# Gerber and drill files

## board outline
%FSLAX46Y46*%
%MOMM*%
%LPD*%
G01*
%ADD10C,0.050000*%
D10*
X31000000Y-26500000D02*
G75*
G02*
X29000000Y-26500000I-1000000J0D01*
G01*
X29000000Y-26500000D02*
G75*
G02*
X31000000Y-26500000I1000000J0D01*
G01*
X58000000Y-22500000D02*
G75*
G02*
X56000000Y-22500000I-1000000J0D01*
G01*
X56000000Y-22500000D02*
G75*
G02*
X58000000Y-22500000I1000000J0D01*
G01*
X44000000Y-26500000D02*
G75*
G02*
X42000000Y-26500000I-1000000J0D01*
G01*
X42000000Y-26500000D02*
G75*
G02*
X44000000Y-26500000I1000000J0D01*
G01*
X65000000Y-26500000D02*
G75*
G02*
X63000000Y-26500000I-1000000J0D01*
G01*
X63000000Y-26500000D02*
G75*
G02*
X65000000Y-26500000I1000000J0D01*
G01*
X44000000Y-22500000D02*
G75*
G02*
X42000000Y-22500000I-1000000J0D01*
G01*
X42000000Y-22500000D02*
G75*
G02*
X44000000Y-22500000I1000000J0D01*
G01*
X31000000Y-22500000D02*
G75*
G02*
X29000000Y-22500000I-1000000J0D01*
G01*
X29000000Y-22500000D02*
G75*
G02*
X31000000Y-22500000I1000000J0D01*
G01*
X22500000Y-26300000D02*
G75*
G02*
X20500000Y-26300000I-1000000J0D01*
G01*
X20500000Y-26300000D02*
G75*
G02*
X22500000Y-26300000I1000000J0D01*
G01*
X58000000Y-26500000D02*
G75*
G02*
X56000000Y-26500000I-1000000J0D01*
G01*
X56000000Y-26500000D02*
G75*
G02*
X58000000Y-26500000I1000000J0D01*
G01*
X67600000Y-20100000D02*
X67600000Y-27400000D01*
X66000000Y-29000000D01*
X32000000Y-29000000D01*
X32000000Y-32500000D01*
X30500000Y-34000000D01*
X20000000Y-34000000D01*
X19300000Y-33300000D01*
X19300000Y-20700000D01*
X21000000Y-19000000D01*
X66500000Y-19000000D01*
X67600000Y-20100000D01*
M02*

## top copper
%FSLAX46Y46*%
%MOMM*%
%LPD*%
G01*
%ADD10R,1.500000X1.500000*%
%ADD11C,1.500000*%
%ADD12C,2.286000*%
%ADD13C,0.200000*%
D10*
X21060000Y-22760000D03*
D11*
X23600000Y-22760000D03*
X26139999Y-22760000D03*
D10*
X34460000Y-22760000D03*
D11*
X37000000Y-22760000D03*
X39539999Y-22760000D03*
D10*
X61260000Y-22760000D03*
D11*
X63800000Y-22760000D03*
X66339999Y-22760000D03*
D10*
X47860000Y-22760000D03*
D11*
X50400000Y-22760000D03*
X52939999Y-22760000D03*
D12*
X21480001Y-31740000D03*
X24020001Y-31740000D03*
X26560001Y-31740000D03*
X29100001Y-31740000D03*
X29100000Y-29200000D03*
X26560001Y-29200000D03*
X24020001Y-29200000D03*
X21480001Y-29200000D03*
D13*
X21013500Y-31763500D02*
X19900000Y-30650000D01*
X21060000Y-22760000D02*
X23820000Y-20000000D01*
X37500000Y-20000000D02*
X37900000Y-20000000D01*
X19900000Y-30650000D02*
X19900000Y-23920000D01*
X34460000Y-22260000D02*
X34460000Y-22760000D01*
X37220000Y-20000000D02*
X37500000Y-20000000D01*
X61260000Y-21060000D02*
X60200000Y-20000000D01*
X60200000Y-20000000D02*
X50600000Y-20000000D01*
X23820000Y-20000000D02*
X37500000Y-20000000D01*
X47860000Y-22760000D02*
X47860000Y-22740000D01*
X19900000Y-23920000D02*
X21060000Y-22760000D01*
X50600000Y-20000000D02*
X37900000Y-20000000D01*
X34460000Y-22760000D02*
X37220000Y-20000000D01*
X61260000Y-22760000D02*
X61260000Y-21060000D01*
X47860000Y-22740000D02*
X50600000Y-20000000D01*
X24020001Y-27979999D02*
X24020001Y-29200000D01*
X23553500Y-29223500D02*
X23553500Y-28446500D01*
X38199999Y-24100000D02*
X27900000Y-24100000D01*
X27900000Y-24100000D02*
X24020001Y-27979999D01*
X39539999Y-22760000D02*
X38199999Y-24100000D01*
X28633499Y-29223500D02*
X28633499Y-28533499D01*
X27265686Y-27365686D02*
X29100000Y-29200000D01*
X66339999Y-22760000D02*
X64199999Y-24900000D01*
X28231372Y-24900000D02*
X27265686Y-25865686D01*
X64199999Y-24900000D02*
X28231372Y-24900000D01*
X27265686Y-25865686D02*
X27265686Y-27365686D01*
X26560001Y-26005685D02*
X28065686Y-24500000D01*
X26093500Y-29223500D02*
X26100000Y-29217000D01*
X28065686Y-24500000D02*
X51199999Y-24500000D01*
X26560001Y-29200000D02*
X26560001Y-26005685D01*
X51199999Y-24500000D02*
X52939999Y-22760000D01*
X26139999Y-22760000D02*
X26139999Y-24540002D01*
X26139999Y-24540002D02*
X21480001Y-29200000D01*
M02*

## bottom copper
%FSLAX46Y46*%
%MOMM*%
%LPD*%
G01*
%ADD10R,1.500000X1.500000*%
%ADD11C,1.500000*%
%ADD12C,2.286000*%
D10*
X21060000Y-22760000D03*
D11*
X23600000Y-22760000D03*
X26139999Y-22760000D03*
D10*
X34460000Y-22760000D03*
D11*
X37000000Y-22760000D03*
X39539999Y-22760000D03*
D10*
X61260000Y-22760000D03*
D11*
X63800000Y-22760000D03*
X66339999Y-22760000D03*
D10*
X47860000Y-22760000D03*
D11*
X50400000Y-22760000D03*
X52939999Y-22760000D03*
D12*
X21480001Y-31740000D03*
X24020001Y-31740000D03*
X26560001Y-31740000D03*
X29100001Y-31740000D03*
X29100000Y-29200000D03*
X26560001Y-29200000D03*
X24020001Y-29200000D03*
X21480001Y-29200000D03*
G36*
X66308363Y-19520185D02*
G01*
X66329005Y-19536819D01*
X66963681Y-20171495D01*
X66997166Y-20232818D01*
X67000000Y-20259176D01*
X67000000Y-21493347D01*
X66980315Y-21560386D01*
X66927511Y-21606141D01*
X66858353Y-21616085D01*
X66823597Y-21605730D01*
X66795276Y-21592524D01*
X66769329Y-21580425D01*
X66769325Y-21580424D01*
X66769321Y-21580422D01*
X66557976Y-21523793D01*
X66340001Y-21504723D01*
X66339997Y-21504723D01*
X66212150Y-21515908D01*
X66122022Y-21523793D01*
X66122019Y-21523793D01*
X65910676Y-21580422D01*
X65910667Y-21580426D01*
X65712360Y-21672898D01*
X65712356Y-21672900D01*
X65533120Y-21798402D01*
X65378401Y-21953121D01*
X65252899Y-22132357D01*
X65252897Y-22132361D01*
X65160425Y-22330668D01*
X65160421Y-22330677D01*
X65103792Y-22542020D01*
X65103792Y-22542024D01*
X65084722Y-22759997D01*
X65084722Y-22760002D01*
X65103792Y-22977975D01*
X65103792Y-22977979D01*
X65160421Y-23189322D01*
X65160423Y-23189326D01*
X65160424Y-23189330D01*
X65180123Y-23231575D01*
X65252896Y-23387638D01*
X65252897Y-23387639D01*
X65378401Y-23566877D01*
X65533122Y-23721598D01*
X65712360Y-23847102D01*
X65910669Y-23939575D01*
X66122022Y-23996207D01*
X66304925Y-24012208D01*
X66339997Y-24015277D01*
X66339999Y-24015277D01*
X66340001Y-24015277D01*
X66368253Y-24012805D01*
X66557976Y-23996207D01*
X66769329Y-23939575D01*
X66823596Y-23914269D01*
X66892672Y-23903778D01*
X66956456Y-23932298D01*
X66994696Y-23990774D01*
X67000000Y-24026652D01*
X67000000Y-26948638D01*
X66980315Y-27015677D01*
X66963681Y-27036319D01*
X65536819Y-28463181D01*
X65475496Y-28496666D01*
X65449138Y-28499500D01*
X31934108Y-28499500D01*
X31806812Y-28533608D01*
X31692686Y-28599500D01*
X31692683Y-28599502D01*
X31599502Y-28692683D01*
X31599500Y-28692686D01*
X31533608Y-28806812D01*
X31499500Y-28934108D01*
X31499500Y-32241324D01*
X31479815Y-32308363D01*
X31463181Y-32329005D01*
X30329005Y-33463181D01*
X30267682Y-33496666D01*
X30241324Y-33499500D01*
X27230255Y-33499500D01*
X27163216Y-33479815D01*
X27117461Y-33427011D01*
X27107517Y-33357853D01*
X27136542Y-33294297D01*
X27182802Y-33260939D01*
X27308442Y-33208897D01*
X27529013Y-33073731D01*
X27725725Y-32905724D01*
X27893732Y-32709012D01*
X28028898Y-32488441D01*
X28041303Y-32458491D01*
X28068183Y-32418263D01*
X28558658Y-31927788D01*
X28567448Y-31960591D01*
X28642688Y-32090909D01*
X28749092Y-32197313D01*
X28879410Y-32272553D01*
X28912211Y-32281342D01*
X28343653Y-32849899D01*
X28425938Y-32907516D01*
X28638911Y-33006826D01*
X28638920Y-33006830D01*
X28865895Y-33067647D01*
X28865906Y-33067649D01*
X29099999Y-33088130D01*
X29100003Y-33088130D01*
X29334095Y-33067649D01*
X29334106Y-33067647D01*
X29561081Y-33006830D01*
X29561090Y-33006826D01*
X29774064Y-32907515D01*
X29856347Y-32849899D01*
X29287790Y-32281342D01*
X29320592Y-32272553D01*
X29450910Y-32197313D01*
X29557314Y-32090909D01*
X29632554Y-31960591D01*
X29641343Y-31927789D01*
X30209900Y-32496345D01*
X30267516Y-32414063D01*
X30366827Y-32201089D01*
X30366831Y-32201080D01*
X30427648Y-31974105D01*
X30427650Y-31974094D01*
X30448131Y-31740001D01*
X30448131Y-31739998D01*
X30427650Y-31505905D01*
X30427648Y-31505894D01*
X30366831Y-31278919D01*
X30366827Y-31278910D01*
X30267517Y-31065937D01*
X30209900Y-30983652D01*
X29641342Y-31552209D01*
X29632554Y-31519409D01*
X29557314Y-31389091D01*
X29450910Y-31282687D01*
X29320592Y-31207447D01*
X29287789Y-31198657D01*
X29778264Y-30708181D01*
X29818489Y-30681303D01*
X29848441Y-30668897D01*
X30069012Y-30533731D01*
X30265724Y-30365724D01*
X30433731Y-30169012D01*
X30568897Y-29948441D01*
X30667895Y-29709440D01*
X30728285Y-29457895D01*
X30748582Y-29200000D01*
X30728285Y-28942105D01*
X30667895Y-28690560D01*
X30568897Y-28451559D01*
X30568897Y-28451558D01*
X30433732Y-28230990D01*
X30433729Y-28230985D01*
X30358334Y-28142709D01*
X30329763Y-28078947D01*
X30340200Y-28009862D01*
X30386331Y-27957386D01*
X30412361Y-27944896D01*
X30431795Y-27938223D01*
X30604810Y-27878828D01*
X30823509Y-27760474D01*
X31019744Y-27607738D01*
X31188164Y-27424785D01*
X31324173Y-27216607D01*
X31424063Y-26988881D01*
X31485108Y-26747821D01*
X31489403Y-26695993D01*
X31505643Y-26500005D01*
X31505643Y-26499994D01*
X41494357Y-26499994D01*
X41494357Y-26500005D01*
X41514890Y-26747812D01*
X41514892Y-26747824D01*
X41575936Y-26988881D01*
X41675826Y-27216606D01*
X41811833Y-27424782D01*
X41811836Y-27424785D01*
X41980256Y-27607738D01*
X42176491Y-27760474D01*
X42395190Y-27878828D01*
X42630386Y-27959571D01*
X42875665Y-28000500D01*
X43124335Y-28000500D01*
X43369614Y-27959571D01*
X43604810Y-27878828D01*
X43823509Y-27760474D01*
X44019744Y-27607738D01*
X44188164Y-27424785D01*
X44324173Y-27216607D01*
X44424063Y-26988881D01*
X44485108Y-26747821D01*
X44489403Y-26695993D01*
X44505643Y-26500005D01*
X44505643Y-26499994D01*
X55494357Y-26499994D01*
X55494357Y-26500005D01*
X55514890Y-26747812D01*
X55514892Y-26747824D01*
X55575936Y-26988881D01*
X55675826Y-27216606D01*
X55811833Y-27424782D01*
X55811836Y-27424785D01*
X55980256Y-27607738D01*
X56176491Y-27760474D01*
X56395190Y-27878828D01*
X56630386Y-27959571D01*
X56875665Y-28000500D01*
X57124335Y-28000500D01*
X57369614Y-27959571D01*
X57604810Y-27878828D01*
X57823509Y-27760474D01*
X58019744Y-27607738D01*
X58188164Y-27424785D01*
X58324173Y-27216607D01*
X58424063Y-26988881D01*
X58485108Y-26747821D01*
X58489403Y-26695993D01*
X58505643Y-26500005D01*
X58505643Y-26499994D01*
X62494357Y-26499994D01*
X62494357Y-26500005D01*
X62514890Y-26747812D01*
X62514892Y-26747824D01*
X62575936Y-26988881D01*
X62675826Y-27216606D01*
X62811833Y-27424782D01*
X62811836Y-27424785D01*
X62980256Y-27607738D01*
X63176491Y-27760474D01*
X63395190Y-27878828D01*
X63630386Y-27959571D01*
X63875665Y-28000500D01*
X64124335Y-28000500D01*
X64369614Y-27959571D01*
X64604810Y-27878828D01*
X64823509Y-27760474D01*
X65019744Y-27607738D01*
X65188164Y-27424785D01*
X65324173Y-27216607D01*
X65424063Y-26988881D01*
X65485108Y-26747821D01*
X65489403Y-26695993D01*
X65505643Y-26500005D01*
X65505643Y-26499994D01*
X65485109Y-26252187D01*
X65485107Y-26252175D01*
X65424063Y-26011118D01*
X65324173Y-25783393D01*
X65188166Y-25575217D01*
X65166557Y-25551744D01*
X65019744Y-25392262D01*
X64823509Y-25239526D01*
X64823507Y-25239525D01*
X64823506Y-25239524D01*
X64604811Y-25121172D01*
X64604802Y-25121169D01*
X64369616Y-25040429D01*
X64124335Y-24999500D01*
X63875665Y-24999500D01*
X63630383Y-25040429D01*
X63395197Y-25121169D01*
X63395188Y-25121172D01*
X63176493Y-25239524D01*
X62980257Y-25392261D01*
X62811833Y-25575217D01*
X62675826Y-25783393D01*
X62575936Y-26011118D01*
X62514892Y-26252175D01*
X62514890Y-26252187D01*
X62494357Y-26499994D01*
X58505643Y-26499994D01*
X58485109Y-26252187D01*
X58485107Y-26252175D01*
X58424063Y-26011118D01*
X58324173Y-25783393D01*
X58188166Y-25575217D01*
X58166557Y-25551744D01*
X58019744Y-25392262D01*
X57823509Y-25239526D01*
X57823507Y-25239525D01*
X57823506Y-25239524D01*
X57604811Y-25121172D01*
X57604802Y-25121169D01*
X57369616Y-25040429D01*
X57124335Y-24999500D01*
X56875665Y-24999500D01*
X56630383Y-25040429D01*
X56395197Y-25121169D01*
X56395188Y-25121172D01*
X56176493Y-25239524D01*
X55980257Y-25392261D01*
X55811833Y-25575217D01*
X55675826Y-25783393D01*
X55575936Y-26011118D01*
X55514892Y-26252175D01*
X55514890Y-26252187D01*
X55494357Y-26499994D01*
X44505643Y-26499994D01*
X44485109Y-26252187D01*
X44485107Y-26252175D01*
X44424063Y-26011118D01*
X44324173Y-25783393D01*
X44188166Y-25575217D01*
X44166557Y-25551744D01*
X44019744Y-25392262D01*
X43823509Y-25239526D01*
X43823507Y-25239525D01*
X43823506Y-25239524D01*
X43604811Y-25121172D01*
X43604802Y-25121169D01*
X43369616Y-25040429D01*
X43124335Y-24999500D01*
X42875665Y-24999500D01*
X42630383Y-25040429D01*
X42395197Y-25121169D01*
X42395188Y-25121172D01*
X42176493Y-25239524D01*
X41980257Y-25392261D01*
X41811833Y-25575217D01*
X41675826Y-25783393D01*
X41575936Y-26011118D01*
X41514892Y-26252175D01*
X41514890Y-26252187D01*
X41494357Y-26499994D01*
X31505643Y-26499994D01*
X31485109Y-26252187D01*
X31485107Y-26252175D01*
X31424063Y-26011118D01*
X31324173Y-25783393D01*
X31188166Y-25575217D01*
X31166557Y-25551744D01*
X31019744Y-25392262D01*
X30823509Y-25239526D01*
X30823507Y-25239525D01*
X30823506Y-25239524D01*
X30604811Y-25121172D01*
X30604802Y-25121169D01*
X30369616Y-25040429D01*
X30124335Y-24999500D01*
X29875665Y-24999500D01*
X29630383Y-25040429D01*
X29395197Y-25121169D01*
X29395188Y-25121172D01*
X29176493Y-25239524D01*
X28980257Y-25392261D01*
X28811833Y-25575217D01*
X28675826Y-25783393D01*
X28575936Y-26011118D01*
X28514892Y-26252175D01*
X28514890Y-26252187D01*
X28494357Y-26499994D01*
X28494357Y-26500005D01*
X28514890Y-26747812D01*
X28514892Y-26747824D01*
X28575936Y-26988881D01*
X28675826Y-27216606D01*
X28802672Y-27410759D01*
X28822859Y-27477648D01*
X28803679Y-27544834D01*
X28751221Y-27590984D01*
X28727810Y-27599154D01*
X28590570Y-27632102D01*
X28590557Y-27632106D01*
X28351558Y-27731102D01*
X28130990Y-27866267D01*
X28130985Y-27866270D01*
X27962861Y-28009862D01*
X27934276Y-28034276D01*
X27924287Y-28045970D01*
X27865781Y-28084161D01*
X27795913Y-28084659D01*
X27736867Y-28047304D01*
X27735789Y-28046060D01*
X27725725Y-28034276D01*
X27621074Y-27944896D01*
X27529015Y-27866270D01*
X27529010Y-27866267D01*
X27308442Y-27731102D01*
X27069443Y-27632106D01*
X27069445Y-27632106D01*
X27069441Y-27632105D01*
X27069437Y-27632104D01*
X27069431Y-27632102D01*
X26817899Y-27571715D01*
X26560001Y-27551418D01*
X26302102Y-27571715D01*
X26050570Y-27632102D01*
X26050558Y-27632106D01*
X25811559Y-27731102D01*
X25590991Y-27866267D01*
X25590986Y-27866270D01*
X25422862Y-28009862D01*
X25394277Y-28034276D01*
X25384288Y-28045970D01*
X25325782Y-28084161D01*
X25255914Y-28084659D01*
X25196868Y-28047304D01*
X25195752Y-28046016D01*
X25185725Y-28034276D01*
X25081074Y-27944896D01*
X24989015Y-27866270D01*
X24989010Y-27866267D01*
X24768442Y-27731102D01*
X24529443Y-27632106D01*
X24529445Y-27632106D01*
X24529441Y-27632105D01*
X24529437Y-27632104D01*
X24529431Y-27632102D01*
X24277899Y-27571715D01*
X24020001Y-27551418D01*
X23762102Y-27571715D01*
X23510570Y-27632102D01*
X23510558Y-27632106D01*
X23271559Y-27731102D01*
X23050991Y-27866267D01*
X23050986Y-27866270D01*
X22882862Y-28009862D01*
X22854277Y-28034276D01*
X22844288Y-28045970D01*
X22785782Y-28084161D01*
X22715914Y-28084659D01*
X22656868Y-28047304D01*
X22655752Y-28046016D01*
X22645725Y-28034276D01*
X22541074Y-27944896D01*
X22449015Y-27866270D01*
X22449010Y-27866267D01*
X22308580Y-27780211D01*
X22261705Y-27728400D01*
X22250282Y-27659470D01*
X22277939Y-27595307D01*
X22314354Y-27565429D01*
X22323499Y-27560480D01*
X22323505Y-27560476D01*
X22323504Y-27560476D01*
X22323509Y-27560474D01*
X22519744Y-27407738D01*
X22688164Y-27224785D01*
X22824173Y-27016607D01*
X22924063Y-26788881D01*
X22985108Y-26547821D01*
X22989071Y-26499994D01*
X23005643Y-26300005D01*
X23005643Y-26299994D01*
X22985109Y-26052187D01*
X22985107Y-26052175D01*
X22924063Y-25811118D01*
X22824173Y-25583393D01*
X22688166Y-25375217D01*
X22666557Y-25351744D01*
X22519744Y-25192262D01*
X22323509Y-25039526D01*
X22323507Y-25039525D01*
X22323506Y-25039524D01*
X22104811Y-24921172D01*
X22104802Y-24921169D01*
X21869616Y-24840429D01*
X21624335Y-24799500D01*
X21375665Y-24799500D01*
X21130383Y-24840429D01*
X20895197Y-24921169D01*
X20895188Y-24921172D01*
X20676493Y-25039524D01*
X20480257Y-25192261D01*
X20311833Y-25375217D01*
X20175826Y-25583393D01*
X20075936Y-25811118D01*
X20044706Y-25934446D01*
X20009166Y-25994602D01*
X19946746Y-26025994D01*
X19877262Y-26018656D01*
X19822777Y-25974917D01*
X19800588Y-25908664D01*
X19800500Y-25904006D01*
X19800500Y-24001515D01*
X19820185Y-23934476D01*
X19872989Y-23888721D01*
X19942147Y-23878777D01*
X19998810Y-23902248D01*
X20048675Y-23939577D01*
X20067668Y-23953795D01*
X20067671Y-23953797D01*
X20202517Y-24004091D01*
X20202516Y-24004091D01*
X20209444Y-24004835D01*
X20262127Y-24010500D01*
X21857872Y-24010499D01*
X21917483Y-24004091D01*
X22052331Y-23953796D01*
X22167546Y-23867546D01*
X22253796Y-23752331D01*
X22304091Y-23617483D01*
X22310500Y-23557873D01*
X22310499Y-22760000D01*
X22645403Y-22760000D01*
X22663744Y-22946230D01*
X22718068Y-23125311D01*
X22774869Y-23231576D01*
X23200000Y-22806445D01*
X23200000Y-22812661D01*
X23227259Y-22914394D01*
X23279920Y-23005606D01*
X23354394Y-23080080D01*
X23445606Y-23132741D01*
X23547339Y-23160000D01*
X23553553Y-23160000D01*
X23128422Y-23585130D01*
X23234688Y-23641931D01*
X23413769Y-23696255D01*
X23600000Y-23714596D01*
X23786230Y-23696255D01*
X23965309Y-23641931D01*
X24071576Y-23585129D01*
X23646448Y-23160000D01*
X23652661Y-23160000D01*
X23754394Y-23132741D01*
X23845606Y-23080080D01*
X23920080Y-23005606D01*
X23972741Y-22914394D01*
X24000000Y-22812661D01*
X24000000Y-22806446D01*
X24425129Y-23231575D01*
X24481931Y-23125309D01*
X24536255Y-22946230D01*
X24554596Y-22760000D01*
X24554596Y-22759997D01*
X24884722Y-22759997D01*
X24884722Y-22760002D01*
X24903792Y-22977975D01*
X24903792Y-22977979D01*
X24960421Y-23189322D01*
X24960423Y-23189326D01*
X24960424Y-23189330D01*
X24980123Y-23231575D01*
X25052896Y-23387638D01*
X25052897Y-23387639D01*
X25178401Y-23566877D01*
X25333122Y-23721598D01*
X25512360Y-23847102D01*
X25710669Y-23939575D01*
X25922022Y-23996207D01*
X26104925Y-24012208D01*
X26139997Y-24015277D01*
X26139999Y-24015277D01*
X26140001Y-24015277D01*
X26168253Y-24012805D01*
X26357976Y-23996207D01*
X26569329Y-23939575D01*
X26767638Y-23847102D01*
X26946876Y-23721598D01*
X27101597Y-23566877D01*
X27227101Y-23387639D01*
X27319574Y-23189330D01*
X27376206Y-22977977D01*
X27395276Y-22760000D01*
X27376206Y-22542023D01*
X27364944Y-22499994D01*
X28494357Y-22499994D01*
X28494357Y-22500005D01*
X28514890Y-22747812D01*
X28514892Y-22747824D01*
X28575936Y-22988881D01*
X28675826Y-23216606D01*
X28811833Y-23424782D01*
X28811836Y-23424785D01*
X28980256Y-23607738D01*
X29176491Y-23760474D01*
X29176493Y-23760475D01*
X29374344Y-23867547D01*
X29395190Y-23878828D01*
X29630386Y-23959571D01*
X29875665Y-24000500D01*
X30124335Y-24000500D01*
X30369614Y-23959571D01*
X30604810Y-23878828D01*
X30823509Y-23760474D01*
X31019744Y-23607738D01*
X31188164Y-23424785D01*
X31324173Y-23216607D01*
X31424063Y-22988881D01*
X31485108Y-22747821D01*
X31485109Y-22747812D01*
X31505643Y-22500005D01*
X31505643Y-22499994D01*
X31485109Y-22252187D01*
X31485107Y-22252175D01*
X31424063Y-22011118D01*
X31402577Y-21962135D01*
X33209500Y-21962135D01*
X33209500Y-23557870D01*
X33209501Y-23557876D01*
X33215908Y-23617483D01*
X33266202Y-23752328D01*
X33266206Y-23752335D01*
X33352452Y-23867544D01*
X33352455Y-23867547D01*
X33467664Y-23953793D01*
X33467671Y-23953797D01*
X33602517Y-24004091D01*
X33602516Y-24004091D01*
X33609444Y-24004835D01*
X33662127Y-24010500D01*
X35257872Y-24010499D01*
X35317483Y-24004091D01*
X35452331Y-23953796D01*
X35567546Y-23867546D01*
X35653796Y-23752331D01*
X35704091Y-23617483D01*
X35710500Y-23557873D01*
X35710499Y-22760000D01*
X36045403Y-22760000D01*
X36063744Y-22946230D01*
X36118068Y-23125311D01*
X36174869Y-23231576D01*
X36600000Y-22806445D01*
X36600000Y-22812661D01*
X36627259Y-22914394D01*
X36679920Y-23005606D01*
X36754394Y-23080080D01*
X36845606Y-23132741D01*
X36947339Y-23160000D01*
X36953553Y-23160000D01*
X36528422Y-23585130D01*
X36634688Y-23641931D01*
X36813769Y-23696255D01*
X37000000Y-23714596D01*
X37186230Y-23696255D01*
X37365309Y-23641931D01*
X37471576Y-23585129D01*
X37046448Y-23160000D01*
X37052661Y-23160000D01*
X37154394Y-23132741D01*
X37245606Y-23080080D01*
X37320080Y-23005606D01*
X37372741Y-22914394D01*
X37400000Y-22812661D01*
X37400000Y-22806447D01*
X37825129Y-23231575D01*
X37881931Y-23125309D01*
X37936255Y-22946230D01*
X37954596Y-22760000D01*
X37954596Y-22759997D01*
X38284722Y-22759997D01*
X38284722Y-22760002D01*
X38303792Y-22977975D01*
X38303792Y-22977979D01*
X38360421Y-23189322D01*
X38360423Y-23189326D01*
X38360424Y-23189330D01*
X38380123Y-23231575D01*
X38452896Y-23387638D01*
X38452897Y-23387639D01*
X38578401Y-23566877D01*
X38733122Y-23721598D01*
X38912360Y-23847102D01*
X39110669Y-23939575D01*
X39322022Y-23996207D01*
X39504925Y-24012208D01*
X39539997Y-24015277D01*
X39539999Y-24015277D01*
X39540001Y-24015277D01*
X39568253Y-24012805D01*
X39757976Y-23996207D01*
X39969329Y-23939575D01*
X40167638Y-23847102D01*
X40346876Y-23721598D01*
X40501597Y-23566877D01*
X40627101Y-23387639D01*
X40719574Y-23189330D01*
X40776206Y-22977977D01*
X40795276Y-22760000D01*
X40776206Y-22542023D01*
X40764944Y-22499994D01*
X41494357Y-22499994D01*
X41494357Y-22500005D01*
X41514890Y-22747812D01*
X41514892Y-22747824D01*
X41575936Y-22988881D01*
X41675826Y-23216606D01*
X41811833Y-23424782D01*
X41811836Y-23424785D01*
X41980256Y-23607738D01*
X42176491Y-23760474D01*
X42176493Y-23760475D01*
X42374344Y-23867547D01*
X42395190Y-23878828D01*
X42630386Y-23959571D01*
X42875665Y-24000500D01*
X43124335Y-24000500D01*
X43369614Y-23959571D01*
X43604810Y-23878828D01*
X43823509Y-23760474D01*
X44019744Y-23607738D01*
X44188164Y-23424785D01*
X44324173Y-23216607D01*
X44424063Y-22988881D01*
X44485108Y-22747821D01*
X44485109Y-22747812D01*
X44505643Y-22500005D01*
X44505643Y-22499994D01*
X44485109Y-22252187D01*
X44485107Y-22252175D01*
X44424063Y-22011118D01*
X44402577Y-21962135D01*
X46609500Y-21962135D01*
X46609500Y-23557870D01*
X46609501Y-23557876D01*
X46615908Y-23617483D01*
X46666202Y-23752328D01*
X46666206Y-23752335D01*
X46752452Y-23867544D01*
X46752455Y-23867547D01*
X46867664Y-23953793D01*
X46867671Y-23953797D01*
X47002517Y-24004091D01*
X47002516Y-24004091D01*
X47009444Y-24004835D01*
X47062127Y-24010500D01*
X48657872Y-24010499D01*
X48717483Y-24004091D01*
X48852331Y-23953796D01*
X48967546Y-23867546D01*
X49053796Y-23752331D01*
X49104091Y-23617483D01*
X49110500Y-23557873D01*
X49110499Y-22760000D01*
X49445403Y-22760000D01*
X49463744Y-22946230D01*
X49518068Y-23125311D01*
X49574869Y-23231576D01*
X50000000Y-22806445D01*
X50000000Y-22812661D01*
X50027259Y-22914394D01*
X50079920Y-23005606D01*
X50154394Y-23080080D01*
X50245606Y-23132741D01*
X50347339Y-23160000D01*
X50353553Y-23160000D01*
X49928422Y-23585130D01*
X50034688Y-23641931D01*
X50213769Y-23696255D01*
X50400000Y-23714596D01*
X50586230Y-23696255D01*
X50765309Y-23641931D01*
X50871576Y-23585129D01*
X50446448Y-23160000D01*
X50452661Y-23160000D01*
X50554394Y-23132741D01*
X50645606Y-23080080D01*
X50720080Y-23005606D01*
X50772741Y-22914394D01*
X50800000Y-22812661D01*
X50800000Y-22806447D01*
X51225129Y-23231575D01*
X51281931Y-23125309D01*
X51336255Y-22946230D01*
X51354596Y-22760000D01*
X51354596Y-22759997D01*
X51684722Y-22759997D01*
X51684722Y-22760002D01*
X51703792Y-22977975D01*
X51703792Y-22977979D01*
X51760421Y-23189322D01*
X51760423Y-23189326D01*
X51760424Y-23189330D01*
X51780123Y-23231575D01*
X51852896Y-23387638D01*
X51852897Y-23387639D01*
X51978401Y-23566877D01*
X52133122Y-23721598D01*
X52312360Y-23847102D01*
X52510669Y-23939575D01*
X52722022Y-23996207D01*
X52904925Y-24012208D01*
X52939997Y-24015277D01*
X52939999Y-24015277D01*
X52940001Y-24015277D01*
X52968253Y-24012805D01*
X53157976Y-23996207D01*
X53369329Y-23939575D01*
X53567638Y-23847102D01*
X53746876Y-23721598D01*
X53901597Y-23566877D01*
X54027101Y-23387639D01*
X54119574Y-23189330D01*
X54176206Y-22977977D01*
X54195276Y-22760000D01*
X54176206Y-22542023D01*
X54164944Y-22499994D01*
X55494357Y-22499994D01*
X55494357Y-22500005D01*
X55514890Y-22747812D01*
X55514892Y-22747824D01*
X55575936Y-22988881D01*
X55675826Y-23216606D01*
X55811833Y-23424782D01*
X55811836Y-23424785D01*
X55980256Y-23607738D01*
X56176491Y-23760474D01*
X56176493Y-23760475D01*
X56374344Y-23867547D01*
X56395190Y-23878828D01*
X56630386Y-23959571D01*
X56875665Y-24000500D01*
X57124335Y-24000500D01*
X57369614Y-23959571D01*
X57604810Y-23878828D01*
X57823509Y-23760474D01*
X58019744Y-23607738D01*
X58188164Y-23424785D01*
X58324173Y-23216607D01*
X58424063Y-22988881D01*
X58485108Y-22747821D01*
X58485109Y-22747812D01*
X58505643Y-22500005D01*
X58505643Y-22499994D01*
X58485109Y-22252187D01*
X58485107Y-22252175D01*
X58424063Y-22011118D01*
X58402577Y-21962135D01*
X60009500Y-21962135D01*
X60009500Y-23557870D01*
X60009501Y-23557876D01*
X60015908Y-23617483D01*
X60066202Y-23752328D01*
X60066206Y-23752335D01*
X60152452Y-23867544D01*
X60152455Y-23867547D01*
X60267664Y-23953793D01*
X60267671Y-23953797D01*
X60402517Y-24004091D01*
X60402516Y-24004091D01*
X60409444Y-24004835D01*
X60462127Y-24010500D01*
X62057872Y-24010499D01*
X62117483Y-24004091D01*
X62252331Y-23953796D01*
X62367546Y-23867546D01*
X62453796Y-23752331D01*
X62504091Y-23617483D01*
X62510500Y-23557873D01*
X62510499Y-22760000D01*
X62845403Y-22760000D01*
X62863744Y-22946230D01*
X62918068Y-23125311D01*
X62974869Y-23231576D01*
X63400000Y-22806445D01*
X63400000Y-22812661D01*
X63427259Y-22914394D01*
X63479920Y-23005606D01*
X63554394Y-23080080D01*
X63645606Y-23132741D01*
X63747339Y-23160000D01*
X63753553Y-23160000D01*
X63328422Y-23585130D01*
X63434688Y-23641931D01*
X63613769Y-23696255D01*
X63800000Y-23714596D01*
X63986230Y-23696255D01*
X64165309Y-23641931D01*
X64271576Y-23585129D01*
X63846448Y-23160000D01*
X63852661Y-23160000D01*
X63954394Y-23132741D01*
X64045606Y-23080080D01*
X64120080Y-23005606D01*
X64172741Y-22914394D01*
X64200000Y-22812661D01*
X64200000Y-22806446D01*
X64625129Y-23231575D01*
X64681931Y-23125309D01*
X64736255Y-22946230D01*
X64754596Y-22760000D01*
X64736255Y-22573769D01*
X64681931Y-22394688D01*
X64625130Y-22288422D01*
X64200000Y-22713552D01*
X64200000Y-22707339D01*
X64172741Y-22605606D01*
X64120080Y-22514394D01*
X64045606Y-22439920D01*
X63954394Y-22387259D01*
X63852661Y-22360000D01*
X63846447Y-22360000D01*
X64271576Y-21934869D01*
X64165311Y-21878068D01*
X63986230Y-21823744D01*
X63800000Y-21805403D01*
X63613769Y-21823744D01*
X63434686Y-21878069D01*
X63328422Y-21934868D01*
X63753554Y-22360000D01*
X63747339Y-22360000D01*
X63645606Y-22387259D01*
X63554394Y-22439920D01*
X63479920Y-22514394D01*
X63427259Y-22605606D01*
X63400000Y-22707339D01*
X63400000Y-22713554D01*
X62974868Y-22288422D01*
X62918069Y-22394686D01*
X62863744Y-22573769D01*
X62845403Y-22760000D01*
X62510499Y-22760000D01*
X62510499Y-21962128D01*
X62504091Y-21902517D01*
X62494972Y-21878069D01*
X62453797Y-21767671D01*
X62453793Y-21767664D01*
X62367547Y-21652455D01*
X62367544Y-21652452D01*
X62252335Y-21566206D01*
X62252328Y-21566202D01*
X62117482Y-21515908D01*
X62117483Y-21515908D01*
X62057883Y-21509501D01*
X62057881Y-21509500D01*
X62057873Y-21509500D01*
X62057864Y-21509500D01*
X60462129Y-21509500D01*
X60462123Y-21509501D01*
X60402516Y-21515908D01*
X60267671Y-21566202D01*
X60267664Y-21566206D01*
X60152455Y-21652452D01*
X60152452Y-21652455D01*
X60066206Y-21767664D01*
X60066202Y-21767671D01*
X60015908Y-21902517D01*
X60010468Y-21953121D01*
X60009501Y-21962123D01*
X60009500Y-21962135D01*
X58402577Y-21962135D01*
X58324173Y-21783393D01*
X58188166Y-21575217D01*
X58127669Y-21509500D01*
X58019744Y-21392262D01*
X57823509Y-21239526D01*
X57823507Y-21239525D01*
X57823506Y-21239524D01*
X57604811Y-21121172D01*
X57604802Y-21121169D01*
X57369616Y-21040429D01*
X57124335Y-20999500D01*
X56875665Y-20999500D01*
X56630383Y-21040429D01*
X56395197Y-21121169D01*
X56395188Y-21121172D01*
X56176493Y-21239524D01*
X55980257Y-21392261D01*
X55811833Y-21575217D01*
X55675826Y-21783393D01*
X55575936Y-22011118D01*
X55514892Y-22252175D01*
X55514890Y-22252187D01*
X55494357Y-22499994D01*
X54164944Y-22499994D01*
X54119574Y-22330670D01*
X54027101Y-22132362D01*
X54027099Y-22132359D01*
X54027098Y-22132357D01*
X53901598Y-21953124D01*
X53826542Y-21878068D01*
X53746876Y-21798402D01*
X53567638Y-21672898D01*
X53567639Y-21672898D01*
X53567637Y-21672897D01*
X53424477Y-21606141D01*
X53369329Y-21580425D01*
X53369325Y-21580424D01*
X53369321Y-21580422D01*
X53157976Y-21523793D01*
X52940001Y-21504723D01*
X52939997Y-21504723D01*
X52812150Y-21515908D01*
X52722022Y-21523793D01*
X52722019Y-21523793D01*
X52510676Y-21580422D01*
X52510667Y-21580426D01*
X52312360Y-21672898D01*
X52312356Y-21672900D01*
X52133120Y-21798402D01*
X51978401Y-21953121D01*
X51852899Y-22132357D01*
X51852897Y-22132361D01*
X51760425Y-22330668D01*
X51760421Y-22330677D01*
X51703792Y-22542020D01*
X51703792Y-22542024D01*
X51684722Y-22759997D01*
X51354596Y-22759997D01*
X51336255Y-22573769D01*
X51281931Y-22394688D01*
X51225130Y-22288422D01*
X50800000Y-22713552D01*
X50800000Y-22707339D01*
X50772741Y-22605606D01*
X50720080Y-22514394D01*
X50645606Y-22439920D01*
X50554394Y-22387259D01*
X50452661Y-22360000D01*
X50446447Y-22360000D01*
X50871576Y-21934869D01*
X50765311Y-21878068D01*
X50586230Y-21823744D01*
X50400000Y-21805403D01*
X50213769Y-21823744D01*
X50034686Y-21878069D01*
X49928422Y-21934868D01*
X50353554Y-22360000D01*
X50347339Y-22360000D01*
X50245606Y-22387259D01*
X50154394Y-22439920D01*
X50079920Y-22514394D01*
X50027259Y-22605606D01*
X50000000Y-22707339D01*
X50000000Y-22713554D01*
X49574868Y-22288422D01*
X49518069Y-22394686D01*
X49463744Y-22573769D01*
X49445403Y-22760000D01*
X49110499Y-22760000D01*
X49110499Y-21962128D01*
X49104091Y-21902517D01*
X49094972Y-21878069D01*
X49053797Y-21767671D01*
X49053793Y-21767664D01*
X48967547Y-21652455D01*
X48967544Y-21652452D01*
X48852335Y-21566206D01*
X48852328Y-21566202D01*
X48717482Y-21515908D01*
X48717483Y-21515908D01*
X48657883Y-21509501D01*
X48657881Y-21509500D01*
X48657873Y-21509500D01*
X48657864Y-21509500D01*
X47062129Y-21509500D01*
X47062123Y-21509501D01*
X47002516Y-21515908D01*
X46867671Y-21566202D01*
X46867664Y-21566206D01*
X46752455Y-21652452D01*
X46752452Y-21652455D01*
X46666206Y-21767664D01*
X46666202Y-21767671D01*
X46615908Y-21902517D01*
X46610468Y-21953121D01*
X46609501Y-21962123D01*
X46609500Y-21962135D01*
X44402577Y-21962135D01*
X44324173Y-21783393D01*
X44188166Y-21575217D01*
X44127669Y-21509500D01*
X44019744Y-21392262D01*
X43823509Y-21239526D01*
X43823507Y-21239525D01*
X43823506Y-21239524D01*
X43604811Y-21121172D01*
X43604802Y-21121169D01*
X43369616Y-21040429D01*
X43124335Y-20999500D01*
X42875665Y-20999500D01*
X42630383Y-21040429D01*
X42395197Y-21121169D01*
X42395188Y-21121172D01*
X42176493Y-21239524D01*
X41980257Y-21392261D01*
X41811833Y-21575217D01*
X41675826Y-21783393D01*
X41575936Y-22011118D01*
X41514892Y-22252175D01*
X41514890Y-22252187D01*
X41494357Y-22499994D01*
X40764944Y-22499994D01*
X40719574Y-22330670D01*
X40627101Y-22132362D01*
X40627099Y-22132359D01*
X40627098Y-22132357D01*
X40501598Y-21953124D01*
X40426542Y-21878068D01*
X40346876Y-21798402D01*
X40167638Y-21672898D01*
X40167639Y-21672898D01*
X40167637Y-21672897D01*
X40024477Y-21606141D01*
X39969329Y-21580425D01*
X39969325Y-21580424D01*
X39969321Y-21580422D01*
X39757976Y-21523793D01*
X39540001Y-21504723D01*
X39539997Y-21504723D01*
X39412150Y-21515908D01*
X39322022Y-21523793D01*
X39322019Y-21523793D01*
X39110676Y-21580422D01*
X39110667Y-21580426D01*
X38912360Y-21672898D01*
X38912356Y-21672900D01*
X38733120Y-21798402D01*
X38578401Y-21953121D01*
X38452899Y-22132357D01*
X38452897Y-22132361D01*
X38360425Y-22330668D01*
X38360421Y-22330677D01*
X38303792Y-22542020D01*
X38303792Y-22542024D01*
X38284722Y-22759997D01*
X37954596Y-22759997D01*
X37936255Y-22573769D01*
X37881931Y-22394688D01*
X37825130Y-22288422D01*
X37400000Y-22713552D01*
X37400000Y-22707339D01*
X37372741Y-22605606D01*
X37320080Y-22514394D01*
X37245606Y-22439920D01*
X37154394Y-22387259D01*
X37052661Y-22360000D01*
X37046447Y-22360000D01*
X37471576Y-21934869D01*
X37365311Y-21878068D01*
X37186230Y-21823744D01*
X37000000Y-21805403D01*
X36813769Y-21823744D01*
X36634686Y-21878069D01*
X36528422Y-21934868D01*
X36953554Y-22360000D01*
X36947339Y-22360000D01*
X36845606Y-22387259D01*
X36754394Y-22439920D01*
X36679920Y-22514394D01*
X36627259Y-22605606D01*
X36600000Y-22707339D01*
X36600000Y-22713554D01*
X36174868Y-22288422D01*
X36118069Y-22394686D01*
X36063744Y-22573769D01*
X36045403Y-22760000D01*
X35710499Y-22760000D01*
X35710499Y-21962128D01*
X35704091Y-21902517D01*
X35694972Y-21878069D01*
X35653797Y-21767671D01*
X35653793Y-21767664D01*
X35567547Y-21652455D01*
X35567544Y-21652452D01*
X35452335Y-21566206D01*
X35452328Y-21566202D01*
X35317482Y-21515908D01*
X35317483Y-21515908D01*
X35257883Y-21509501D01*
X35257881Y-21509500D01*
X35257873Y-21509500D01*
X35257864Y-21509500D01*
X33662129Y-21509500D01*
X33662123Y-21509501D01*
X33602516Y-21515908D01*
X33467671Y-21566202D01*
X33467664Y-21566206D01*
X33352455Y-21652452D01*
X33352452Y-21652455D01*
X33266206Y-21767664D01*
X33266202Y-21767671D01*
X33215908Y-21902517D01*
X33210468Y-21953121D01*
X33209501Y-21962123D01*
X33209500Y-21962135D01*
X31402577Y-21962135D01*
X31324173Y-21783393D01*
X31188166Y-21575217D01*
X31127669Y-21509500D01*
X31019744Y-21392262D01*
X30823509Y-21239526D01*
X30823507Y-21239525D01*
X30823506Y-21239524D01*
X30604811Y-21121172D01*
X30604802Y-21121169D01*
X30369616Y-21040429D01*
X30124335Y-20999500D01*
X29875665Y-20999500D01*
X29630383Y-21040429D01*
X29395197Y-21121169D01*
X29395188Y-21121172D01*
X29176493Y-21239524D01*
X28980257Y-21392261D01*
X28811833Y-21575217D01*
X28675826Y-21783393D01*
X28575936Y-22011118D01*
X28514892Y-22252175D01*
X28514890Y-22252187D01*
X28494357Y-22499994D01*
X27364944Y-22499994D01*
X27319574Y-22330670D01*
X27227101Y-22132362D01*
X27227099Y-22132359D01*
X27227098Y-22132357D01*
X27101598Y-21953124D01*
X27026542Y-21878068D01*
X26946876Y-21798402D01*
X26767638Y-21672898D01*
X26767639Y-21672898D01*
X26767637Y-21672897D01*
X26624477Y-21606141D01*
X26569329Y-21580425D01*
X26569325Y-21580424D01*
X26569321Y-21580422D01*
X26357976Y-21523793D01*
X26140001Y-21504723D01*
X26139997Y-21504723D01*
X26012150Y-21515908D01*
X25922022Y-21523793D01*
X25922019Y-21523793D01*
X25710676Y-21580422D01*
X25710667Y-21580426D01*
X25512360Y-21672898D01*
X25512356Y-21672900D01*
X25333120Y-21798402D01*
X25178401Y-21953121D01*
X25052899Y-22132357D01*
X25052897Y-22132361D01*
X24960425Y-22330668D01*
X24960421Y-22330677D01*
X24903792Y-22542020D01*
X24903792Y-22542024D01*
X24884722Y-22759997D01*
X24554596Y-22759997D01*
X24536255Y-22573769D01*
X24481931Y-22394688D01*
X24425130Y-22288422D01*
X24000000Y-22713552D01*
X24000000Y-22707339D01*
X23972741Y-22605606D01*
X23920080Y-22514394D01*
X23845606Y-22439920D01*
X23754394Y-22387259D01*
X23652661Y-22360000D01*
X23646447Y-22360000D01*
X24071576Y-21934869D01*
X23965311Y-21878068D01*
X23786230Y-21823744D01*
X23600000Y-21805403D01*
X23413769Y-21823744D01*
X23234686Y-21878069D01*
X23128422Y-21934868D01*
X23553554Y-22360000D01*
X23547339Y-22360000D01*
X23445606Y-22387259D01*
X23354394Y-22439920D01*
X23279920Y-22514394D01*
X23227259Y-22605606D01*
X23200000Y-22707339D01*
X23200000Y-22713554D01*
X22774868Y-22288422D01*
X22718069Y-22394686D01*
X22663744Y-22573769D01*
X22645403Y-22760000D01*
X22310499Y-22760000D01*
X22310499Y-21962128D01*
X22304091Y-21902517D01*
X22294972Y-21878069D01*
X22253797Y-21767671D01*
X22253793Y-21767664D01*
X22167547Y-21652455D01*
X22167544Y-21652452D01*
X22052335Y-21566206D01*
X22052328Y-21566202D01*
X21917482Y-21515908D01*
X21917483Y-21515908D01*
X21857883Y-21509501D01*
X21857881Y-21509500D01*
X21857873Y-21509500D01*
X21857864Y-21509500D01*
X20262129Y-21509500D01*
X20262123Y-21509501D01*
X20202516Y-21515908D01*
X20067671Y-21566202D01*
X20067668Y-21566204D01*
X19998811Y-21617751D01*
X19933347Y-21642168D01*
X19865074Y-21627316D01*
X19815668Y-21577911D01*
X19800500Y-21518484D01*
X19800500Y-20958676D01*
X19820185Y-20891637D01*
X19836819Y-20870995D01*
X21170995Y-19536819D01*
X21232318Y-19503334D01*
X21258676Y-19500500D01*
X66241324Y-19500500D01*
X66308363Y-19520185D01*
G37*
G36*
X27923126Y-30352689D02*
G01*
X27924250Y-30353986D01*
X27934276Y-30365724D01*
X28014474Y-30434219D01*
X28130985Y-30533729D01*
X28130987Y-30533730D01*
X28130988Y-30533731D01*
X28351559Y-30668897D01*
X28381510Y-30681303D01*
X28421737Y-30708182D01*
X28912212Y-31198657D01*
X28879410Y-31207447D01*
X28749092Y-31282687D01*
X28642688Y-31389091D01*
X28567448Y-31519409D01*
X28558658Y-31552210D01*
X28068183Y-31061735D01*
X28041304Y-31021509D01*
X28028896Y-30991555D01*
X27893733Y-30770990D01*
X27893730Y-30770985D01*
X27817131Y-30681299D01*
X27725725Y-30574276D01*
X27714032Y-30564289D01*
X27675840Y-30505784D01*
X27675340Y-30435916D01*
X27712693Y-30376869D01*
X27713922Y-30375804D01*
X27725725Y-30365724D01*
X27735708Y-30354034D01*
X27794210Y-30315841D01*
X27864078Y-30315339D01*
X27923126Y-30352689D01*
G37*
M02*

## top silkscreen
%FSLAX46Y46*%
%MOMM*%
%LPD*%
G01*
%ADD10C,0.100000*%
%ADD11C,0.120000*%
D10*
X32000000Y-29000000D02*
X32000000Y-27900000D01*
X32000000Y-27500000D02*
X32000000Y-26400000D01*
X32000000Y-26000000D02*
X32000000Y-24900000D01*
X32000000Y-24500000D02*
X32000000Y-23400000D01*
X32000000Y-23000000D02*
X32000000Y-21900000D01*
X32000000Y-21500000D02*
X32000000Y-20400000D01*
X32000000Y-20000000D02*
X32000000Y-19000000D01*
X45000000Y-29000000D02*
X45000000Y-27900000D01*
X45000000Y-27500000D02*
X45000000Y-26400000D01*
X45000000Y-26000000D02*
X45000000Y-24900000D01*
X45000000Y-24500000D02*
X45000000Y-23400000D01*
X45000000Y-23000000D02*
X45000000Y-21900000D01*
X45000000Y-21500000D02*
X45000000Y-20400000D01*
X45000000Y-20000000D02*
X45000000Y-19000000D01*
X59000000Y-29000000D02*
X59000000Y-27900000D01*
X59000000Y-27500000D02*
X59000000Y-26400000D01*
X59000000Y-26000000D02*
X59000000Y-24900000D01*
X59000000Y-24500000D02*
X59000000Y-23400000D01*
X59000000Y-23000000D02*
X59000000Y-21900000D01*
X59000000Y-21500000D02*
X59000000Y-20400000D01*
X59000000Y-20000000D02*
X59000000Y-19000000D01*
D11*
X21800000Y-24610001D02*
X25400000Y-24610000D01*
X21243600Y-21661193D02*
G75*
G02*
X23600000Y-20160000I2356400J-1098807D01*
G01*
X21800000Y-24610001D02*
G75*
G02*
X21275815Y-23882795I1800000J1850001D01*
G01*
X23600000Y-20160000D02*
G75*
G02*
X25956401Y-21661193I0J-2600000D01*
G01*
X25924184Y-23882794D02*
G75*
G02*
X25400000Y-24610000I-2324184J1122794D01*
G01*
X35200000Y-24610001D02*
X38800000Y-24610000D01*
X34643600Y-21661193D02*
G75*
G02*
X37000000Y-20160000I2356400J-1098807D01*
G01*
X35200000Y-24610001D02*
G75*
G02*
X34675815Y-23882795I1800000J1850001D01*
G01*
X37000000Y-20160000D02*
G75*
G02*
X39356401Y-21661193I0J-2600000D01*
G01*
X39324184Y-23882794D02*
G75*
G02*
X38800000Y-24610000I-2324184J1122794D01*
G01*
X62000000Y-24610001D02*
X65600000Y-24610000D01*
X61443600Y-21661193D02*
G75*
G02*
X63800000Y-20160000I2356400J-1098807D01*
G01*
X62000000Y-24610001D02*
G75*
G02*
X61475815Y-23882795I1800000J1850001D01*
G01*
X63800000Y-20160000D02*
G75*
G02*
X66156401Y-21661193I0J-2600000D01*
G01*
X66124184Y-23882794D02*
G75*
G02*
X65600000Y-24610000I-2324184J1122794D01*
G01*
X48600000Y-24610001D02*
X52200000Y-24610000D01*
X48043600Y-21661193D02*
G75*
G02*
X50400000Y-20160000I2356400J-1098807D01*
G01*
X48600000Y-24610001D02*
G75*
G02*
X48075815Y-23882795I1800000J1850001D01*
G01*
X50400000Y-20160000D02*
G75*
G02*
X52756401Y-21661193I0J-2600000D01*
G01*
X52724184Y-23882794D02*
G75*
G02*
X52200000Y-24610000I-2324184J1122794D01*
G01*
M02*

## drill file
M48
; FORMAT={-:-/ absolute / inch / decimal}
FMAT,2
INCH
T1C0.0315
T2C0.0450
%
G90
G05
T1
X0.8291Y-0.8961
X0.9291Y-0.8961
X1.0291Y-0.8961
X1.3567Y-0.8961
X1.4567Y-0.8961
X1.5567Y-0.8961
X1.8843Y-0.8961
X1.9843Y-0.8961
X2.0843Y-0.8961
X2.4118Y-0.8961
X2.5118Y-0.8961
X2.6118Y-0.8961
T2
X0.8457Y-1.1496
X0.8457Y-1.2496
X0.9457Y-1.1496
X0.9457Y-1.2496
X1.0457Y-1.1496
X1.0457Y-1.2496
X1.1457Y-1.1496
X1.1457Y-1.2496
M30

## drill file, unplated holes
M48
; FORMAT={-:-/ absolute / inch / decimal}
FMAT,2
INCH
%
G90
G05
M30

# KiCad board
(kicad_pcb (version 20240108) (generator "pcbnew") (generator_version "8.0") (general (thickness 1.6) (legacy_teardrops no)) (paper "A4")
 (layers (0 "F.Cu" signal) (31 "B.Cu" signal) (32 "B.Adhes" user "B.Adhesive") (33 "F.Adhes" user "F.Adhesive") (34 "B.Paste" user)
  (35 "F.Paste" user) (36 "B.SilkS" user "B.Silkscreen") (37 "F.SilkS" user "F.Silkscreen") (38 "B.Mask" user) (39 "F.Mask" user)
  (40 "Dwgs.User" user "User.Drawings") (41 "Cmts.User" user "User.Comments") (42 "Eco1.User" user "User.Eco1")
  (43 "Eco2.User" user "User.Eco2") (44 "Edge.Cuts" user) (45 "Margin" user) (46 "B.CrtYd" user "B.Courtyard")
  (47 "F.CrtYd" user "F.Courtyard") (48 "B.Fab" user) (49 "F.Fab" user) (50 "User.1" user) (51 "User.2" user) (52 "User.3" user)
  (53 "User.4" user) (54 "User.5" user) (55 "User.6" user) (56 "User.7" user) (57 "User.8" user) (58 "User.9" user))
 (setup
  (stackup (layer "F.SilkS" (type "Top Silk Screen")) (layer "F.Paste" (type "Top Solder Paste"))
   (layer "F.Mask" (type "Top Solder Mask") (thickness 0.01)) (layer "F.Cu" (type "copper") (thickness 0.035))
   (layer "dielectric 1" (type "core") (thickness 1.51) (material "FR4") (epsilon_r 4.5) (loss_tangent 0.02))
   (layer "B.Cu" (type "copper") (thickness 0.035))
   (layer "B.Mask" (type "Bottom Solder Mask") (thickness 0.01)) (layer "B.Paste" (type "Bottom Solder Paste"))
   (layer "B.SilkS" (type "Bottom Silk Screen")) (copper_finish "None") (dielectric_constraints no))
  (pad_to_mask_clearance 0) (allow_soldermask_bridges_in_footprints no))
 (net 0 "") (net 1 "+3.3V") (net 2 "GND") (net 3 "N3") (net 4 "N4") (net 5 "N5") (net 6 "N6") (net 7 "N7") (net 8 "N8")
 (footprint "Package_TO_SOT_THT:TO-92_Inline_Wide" (layer "F.Cu") (at 21.06 22.76)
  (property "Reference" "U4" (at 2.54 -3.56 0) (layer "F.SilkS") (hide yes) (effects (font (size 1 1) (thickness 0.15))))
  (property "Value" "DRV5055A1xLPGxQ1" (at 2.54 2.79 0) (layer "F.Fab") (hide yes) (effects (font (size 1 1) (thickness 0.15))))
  (fp_line (start 0.74 1.850001) (end 4.34 1.85) (stroke (width 0.12) (type solid)) (layer "F.SilkS"))
  (fp_arc (start 0.1836 -1.098807) (mid 1.143021 -2.192817) (end 2.54 -2.6) (stroke (width 0.12) (type solid)) (layer "F.SilkS"))
  (fp_arc (start 0.74 1.850001) (mid 0.446097 1.509328) (end 0.215816 1.122795) (stroke (width 0.12) (type solid)) (layer "F.SilkS"))
  (fp_arc (start 2.54 -2.6) (mid 3.936979 -2.192818) (end 4.896401 -1.098807) (stroke (width 0.12) (type solid)) (layer "F.SilkS"))
  (fp_arc (start 4.864184 1.122794) (mid 4.633903 1.509327) (end 4.34 1.85) (stroke (width 0.12) (type solid)) (layer "F.SilkS"))
  (pad "1" thru_hole rect (at 0 0) (size 1.5 1.5) (drill 0.8) (layers "*.Cu" "*.Mask") (remove_unused_layers no) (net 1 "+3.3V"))
  (pad "2" thru_hole circle (at 2.54 0) (size 1.5 1.5) (drill 0.8) (layers "*.Cu" "*.Mask") (remove_unused_layers no) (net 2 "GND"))
  (pad "3" thru_hole circle (at 5.079999 0) (size 1.5 1.5) (drill 0.8) (layers "*.Cu" "*.Mask") (remove_unused_layers no) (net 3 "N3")))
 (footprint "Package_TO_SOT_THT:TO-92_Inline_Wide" (layer "F.Cu") (at 34.46 22.76)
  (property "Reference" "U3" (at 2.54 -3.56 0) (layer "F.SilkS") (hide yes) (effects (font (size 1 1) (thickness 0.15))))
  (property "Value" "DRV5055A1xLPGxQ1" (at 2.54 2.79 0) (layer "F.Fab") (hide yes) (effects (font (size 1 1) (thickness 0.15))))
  (fp_line (start 0.74 1.850001) (end 4.34 1.85) (stroke (width 0.12) (type solid)) (layer "F.SilkS"))
  (fp_arc (start 0.1836 -1.098807) (mid 1.143021 -2.192817) (end 2.54 -2.6) (stroke (width 0.12) (type solid)) (layer "F.SilkS"))
  (fp_arc (start 0.74 1.850001) (mid 0.446097 1.509328) (end 0.215816 1.122795) (stroke (width 0.12) (type solid)) (layer "F.SilkS"))
  (fp_arc (start 2.54 -2.6) (mid 3.936979 -2.192818) (end 4.896401 -1.098807) (stroke (width 0.12) (type solid)) (layer "F.SilkS"))
  (fp_arc (start 4.864184 1.122794) (mid 4.633903 1.509327) (end 4.34 1.85) (stroke (width 0.12) (type solid)) (layer "F.SilkS"))
  (pad "1" thru_hole rect (at 0 0) (size 1.5 1.5) (drill 0.8) (layers "*.Cu" "*.Mask") (remove_unused_layers no) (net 1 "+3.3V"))
  (pad "2" thru_hole circle (at 2.54 0) (size 1.5 1.5) (drill 0.8) (layers "*.Cu" "*.Mask") (remove_unused_layers no) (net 2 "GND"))
  (pad "3" thru_hole circle (at 5.079999 0) (size 1.5 1.5) (drill 0.8) (layers "*.Cu" "*.Mask") (remove_unused_layers no) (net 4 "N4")))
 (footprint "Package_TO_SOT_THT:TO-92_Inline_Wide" (layer "F.Cu") (at 61.26 22.76)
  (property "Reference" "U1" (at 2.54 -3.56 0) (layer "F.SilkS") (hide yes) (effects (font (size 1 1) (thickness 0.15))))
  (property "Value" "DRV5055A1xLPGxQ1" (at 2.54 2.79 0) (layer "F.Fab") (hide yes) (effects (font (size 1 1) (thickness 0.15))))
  (fp_line (start 0.74 1.850001) (end 4.34 1.85) (stroke (width 0.12) (type solid)) (layer "F.SilkS"))
  (fp_arc (start 0.1836 -1.098807) (mid 1.143021 -2.192817) (end 2.54 -2.6) (stroke (width 0.12) (type solid)) (layer "F.SilkS"))
  (fp_arc (start 0.74 1.850001) (mid 0.446097 1.509328) (end 0.215816 1.122795) (stroke (width 0.12) (type solid)) (layer "F.SilkS"))
  (fp_arc (start 2.54 -2.6) (mid 3.936979 -2.192818) (end 4.896401 -1.098807) (stroke (width 0.12) (type solid)) (layer "F.SilkS"))
  (fp_arc (start 4.864184 1.122794) (mid 4.633903 1.509327) (end 4.34 1.85) (stroke (width 0.12) (type solid)) (layer "F.SilkS"))
  (pad "1" thru_hole rect (at 0 0) (size 1.5 1.5) (drill 0.8) (layers "*.Cu" "*.Mask") (remove_unused_layers no) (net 1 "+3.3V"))
  (pad "2" thru_hole circle (at 2.54 0) (size 1.5 1.5) (drill 0.8) (layers "*.Cu" "*.Mask") (remove_unused_layers no) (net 2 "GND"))
  (pad "3" thru_hole circle (at 5.079999 0) (size 1.5 1.5) (drill 0.8) (layers "*.Cu" "*.Mask") (remove_unused_layers no) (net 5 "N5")))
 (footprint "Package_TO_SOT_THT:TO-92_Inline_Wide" (layer "F.Cu") (at 47.86 22.76)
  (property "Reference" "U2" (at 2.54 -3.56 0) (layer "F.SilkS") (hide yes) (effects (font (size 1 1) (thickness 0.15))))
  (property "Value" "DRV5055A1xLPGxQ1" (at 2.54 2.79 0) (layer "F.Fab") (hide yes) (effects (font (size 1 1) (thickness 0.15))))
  (fp_line (start 0.74 1.850001) (end 4.34 1.85) (stroke (width 0.12) (type solid)) (layer "F.SilkS"))
  (fp_arc (start 0.1836 -1.098807) (mid 1.143021 -2.192817) (end 2.54 -2.6) (stroke (width 0.12) (type solid)) (layer "F.SilkS"))
  (fp_arc (start 0.74 1.850001) (mid 0.446097 1.509328) (end 0.215816 1.122795) (stroke (width 0.12) (type solid)) (layer "F.SilkS"))
  (fp_arc (start 2.54 -2.6) (mid 3.936979 -2.192818) (end 4.896401 -1.098807) (stroke (width 0.12) (type solid)) (layer "F.SilkS"))
  (fp_arc (start 4.864184 1.122794) (mid 4.633903 1.509327) (end 4.34 1.85) (stroke (width 0.12) (type solid)) (layer "F.SilkS"))
  (pad "1" thru_hole rect (at 0 0) (size 1.5 1.5) (drill 0.8) (layers "*.Cu" "*.Mask") (remove_unused_layers no) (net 1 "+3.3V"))
  (pad "2" thru_hole circle (at 2.54 0) (size 1.5 1.5) (drill 0.8) (layers "*.Cu" "*.Mask") (remove_unused_layers no) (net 2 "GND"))
  (pad "3" thru_hole circle (at 5.079999 0) (size 1.5 1.5) (drill 0.8) (layers "*.Cu" "*.Mask") (remove_unused_layers no) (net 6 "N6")))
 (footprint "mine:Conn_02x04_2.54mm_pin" (layer "F.Cu") (at 18.940001 24.12)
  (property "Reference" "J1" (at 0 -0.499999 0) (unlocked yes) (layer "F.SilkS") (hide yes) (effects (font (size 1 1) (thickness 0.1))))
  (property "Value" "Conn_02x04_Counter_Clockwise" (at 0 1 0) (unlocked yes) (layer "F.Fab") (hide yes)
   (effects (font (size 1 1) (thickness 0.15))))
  (pad "1" thru_hole circle (at 2.54 7.62) (size 2.286 2.286) (drill 1.143) (layers "*.Cu" "*.Mask") (remove_unused_layers no)
   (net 1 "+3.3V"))
  (pad "2" thru_hole circle (at 5.08 7.62) (size 2.286 2.286) (drill 1.143) (layers "*.Cu" "*.Mask") (remove_unused_layers no) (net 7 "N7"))
  (pad "3" thru_hole circle (at 7.62 7.62) (size 2.286 2.286) (drill 1.143) (layers "*.Cu" "*.Mask") (remove_unused_layers no) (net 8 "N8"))
  (pad "4" thru_hole circle (at 10.16 7.62) (size 2.286 2.286) (drill 1.143) (layers "*.Cu" "*.Mask") (remove_unused_layers no)
   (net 2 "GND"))
  (pad "5" thru_hole circle (at 10.159999 5.08) (size 2.286 2.286) (drill 1.143) (layers "*.Cu" "*.Mask") (remove_unused_layers no)
   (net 5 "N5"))
  (pad "6" thru_hole circle (at 7.62 5.08) (size 2.286 2.286) (drill 1.143) (layers "*.Cu" "*.Mask") (remove_unused_layers no) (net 6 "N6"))
  (pad "7" thru_hole circle (at 5.08 5.08) (size 2.286 2.286) (drill 1.143) (layers "*.Cu" "*.Mask") (remove_unused_layers no) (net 4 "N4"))
  (pad "8" thru_hole circle (at 2.54 5.08) (size 2.286 2.286) (drill 1.143) (layers "*.Cu" "*.Mask") (remove_unused_layers no) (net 3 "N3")))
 (gr_line (start 32 29) (end 32 19) (stroke (width 0.1) (type dash)) (layer "F.SilkS"))
 (gr_line (start 45 29) (end 45 19) (stroke (width 0.1) (type dash)) (layer "F.SilkS"))
 (gr_line (start 59 29) (end 59 19) (stroke (width 0.1) (type dash)) (layer "F.SilkS"))
 (gr_circle (center 30 26.5) (end 31 26.5) (stroke (width 0.05) (type default)) (fill none) (layer "Edge.Cuts"))
 (gr_circle (center 57 22.5) (end 58 22.5) (stroke (width 0.05) (type default)) (fill none) (layer "Edge.Cuts"))
 (gr_circle (center 43 26.5) (end 44 26.5) (stroke (width 0.05) (type default)) (fill none) (layer "Edge.Cuts"))
 (gr_circle (center 64 26.5) (end 65 26.5) (stroke (width 0.05) (type default)) (fill none) (layer "Edge.Cuts"))
 (gr_circle (center 43 22.5) (end 44 22.5) (stroke (width 0.05) (type default)) (fill none) (layer "Edge.Cuts"))
 (gr_circle (center 30 22.5) (end 31 22.5) (stroke (width 0.05) (type default)) (fill none) (layer "Edge.Cuts"))
 (gr_circle (center 21.5 26.3) (end 22.5 26.3) (stroke (width 0.05) (type default)) (fill none) (layer "Edge.Cuts"))
 (gr_circle (center 57 26.5) (end 58 26.5) (stroke (width 0.05) (type default)) (fill none) (layer "Edge.Cuts"))
 (gr_poly
  (pts (xy 19.3 20.7) (xy 21 19) (xy 66.5 19) (xy 67.6 20.1) (xy 67.6 27.4) (xy 66 29) (xy 32 29) (xy 32 32.5) (xy 30.5 34) (xy 20 34)
   (xy 19.3 33.3))
  (stroke (width 0.05) (type solid)) (fill none) (layer "Edge.Cuts"))
 (segment (start 21.0135 31.7635) (end 19.9 30.65) (width 0.2) (layer "F.Cu") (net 1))
 (segment (start 21.06 22.76) (end 23.82 20) (width 0.2) (layer "F.Cu") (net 1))
 (segment (start 37.5 20) (end 37.9 20) (width 0.2) (layer "F.Cu") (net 1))
 (segment (start 19.9 30.65) (end 19.9 23.92) (width 0.2) (layer "F.Cu") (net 1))
 (segment (start 34.46 22.26) (end 34.46 22.76) (width 0.2) (layer "F.Cu") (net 1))
 (segment (start 37.22 20) (end 37.5 20) (width 0.2) (layer "F.Cu") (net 1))
 (segment (start 61.26 21.06) (end 60.2 20) (width 0.2) (layer "F.Cu") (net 1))
 (segment (start 60.2 20) (end 50.6 20) (width 0.2) (layer "F.Cu") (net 1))
 (segment (start 23.82 20) (end 37.5 20) (width 0.2) (layer "F.Cu") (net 1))
 (segment (start 47.86 22.76) (end 47.86 22.74) (width 0.2) (layer "F.Cu") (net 1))
 (segment (start 19.9 23.92) (end 21.06 22.76) (width 0.2) (layer "F.Cu") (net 1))
 (segment (start 50.6 20) (end 37.9 20) (width 0.2) (layer "F.Cu") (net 1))
 (segment (start 34.46 22.76) (end 37.22 20) (width 0.2) (layer "F.Cu") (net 1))
 (segment (start 61.26 22.76) (end 61.26 21.06) (width 0.2) (layer "F.Cu") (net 1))
 (segment (start 47.86 22.74) (end 50.6 20) (width 0.2) (layer "F.Cu") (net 1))
 (segment (start 24.020001 27.979999) (end 24.020001 29.2) (width 0.2) (layer "F.Cu") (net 4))
 (segment (start 23.5535 29.2235) (end 23.5535 28.4465) (width 0.2) (layer "F.Cu") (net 4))
 (segment (start 38.199999 24.1) (end 27.9 24.1) (width 0.2) (layer "F.Cu") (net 4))
 (segment (start 27.9 24.1) (end 24.020001 27.979999) (width 0.2) (layer "F.Cu") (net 4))
 (segment (start 39.539999 22.76) (end 38.199999 24.1) (width 0.2) (layer "F.Cu") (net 4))
 (segment (start 28.633499 29.2235) (end 28.633499 28.533499) (width 0.2) (layer "F.Cu") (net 5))
 (segment (start 27.265686 27.365686) (end 29.1 29.2) (width 0.2) (layer "F.Cu") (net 5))
 (segment (start 66.339999 22.76) (end 64.199999 24.9) (width 0.2) (layer "F.Cu") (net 5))
 (segment (start 28.231372 24.9) (end 27.265686 25.865686) (width 0.2) (layer "F.Cu") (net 5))
 (segment (start 64.199999 24.9) (end 28.231372 24.9) (width 0.2) (layer "F.Cu") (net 5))
 (segment (start 27.265686 25.865686) (end 27.265686 27.365686) (width 0.2) (layer "F.Cu") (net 5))
 (segment (start 26.560001 26.005685) (end 28.065686 24.5) (width 0.2) (layer "F.Cu") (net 6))
 (segment (start 26.0935 29.2235) (end 26.1 29.217) (width 0.2) (layer "F.Cu") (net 6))
 (segment (start 28.065686 24.5) (end 51.199999 24.5) (width 0.2) (layer "F.Cu") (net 6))
 (segment (start 26.560001 29.2) (end 26.560001 26.005685) (width 0.2) (layer "F.Cu") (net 6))
 (segment (start 51.199999 24.5) (end 52.939999 22.76) (width 0.2) (layer "F.Cu") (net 6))
 (segment (start 26.139999 22.76) (end 26.139999 24.540002) (width 0.2) (layer "F.Cu") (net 3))
 (segment (start 26.139999 24.540002) (end 21.480001 29.2) (width 0.2) (layer "F.Cu") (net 3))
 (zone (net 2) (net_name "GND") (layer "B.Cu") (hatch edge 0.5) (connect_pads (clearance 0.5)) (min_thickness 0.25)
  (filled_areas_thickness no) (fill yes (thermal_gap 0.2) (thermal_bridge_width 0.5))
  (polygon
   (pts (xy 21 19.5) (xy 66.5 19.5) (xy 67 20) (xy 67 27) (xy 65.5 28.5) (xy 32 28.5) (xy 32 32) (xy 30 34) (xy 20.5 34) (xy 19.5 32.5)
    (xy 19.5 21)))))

